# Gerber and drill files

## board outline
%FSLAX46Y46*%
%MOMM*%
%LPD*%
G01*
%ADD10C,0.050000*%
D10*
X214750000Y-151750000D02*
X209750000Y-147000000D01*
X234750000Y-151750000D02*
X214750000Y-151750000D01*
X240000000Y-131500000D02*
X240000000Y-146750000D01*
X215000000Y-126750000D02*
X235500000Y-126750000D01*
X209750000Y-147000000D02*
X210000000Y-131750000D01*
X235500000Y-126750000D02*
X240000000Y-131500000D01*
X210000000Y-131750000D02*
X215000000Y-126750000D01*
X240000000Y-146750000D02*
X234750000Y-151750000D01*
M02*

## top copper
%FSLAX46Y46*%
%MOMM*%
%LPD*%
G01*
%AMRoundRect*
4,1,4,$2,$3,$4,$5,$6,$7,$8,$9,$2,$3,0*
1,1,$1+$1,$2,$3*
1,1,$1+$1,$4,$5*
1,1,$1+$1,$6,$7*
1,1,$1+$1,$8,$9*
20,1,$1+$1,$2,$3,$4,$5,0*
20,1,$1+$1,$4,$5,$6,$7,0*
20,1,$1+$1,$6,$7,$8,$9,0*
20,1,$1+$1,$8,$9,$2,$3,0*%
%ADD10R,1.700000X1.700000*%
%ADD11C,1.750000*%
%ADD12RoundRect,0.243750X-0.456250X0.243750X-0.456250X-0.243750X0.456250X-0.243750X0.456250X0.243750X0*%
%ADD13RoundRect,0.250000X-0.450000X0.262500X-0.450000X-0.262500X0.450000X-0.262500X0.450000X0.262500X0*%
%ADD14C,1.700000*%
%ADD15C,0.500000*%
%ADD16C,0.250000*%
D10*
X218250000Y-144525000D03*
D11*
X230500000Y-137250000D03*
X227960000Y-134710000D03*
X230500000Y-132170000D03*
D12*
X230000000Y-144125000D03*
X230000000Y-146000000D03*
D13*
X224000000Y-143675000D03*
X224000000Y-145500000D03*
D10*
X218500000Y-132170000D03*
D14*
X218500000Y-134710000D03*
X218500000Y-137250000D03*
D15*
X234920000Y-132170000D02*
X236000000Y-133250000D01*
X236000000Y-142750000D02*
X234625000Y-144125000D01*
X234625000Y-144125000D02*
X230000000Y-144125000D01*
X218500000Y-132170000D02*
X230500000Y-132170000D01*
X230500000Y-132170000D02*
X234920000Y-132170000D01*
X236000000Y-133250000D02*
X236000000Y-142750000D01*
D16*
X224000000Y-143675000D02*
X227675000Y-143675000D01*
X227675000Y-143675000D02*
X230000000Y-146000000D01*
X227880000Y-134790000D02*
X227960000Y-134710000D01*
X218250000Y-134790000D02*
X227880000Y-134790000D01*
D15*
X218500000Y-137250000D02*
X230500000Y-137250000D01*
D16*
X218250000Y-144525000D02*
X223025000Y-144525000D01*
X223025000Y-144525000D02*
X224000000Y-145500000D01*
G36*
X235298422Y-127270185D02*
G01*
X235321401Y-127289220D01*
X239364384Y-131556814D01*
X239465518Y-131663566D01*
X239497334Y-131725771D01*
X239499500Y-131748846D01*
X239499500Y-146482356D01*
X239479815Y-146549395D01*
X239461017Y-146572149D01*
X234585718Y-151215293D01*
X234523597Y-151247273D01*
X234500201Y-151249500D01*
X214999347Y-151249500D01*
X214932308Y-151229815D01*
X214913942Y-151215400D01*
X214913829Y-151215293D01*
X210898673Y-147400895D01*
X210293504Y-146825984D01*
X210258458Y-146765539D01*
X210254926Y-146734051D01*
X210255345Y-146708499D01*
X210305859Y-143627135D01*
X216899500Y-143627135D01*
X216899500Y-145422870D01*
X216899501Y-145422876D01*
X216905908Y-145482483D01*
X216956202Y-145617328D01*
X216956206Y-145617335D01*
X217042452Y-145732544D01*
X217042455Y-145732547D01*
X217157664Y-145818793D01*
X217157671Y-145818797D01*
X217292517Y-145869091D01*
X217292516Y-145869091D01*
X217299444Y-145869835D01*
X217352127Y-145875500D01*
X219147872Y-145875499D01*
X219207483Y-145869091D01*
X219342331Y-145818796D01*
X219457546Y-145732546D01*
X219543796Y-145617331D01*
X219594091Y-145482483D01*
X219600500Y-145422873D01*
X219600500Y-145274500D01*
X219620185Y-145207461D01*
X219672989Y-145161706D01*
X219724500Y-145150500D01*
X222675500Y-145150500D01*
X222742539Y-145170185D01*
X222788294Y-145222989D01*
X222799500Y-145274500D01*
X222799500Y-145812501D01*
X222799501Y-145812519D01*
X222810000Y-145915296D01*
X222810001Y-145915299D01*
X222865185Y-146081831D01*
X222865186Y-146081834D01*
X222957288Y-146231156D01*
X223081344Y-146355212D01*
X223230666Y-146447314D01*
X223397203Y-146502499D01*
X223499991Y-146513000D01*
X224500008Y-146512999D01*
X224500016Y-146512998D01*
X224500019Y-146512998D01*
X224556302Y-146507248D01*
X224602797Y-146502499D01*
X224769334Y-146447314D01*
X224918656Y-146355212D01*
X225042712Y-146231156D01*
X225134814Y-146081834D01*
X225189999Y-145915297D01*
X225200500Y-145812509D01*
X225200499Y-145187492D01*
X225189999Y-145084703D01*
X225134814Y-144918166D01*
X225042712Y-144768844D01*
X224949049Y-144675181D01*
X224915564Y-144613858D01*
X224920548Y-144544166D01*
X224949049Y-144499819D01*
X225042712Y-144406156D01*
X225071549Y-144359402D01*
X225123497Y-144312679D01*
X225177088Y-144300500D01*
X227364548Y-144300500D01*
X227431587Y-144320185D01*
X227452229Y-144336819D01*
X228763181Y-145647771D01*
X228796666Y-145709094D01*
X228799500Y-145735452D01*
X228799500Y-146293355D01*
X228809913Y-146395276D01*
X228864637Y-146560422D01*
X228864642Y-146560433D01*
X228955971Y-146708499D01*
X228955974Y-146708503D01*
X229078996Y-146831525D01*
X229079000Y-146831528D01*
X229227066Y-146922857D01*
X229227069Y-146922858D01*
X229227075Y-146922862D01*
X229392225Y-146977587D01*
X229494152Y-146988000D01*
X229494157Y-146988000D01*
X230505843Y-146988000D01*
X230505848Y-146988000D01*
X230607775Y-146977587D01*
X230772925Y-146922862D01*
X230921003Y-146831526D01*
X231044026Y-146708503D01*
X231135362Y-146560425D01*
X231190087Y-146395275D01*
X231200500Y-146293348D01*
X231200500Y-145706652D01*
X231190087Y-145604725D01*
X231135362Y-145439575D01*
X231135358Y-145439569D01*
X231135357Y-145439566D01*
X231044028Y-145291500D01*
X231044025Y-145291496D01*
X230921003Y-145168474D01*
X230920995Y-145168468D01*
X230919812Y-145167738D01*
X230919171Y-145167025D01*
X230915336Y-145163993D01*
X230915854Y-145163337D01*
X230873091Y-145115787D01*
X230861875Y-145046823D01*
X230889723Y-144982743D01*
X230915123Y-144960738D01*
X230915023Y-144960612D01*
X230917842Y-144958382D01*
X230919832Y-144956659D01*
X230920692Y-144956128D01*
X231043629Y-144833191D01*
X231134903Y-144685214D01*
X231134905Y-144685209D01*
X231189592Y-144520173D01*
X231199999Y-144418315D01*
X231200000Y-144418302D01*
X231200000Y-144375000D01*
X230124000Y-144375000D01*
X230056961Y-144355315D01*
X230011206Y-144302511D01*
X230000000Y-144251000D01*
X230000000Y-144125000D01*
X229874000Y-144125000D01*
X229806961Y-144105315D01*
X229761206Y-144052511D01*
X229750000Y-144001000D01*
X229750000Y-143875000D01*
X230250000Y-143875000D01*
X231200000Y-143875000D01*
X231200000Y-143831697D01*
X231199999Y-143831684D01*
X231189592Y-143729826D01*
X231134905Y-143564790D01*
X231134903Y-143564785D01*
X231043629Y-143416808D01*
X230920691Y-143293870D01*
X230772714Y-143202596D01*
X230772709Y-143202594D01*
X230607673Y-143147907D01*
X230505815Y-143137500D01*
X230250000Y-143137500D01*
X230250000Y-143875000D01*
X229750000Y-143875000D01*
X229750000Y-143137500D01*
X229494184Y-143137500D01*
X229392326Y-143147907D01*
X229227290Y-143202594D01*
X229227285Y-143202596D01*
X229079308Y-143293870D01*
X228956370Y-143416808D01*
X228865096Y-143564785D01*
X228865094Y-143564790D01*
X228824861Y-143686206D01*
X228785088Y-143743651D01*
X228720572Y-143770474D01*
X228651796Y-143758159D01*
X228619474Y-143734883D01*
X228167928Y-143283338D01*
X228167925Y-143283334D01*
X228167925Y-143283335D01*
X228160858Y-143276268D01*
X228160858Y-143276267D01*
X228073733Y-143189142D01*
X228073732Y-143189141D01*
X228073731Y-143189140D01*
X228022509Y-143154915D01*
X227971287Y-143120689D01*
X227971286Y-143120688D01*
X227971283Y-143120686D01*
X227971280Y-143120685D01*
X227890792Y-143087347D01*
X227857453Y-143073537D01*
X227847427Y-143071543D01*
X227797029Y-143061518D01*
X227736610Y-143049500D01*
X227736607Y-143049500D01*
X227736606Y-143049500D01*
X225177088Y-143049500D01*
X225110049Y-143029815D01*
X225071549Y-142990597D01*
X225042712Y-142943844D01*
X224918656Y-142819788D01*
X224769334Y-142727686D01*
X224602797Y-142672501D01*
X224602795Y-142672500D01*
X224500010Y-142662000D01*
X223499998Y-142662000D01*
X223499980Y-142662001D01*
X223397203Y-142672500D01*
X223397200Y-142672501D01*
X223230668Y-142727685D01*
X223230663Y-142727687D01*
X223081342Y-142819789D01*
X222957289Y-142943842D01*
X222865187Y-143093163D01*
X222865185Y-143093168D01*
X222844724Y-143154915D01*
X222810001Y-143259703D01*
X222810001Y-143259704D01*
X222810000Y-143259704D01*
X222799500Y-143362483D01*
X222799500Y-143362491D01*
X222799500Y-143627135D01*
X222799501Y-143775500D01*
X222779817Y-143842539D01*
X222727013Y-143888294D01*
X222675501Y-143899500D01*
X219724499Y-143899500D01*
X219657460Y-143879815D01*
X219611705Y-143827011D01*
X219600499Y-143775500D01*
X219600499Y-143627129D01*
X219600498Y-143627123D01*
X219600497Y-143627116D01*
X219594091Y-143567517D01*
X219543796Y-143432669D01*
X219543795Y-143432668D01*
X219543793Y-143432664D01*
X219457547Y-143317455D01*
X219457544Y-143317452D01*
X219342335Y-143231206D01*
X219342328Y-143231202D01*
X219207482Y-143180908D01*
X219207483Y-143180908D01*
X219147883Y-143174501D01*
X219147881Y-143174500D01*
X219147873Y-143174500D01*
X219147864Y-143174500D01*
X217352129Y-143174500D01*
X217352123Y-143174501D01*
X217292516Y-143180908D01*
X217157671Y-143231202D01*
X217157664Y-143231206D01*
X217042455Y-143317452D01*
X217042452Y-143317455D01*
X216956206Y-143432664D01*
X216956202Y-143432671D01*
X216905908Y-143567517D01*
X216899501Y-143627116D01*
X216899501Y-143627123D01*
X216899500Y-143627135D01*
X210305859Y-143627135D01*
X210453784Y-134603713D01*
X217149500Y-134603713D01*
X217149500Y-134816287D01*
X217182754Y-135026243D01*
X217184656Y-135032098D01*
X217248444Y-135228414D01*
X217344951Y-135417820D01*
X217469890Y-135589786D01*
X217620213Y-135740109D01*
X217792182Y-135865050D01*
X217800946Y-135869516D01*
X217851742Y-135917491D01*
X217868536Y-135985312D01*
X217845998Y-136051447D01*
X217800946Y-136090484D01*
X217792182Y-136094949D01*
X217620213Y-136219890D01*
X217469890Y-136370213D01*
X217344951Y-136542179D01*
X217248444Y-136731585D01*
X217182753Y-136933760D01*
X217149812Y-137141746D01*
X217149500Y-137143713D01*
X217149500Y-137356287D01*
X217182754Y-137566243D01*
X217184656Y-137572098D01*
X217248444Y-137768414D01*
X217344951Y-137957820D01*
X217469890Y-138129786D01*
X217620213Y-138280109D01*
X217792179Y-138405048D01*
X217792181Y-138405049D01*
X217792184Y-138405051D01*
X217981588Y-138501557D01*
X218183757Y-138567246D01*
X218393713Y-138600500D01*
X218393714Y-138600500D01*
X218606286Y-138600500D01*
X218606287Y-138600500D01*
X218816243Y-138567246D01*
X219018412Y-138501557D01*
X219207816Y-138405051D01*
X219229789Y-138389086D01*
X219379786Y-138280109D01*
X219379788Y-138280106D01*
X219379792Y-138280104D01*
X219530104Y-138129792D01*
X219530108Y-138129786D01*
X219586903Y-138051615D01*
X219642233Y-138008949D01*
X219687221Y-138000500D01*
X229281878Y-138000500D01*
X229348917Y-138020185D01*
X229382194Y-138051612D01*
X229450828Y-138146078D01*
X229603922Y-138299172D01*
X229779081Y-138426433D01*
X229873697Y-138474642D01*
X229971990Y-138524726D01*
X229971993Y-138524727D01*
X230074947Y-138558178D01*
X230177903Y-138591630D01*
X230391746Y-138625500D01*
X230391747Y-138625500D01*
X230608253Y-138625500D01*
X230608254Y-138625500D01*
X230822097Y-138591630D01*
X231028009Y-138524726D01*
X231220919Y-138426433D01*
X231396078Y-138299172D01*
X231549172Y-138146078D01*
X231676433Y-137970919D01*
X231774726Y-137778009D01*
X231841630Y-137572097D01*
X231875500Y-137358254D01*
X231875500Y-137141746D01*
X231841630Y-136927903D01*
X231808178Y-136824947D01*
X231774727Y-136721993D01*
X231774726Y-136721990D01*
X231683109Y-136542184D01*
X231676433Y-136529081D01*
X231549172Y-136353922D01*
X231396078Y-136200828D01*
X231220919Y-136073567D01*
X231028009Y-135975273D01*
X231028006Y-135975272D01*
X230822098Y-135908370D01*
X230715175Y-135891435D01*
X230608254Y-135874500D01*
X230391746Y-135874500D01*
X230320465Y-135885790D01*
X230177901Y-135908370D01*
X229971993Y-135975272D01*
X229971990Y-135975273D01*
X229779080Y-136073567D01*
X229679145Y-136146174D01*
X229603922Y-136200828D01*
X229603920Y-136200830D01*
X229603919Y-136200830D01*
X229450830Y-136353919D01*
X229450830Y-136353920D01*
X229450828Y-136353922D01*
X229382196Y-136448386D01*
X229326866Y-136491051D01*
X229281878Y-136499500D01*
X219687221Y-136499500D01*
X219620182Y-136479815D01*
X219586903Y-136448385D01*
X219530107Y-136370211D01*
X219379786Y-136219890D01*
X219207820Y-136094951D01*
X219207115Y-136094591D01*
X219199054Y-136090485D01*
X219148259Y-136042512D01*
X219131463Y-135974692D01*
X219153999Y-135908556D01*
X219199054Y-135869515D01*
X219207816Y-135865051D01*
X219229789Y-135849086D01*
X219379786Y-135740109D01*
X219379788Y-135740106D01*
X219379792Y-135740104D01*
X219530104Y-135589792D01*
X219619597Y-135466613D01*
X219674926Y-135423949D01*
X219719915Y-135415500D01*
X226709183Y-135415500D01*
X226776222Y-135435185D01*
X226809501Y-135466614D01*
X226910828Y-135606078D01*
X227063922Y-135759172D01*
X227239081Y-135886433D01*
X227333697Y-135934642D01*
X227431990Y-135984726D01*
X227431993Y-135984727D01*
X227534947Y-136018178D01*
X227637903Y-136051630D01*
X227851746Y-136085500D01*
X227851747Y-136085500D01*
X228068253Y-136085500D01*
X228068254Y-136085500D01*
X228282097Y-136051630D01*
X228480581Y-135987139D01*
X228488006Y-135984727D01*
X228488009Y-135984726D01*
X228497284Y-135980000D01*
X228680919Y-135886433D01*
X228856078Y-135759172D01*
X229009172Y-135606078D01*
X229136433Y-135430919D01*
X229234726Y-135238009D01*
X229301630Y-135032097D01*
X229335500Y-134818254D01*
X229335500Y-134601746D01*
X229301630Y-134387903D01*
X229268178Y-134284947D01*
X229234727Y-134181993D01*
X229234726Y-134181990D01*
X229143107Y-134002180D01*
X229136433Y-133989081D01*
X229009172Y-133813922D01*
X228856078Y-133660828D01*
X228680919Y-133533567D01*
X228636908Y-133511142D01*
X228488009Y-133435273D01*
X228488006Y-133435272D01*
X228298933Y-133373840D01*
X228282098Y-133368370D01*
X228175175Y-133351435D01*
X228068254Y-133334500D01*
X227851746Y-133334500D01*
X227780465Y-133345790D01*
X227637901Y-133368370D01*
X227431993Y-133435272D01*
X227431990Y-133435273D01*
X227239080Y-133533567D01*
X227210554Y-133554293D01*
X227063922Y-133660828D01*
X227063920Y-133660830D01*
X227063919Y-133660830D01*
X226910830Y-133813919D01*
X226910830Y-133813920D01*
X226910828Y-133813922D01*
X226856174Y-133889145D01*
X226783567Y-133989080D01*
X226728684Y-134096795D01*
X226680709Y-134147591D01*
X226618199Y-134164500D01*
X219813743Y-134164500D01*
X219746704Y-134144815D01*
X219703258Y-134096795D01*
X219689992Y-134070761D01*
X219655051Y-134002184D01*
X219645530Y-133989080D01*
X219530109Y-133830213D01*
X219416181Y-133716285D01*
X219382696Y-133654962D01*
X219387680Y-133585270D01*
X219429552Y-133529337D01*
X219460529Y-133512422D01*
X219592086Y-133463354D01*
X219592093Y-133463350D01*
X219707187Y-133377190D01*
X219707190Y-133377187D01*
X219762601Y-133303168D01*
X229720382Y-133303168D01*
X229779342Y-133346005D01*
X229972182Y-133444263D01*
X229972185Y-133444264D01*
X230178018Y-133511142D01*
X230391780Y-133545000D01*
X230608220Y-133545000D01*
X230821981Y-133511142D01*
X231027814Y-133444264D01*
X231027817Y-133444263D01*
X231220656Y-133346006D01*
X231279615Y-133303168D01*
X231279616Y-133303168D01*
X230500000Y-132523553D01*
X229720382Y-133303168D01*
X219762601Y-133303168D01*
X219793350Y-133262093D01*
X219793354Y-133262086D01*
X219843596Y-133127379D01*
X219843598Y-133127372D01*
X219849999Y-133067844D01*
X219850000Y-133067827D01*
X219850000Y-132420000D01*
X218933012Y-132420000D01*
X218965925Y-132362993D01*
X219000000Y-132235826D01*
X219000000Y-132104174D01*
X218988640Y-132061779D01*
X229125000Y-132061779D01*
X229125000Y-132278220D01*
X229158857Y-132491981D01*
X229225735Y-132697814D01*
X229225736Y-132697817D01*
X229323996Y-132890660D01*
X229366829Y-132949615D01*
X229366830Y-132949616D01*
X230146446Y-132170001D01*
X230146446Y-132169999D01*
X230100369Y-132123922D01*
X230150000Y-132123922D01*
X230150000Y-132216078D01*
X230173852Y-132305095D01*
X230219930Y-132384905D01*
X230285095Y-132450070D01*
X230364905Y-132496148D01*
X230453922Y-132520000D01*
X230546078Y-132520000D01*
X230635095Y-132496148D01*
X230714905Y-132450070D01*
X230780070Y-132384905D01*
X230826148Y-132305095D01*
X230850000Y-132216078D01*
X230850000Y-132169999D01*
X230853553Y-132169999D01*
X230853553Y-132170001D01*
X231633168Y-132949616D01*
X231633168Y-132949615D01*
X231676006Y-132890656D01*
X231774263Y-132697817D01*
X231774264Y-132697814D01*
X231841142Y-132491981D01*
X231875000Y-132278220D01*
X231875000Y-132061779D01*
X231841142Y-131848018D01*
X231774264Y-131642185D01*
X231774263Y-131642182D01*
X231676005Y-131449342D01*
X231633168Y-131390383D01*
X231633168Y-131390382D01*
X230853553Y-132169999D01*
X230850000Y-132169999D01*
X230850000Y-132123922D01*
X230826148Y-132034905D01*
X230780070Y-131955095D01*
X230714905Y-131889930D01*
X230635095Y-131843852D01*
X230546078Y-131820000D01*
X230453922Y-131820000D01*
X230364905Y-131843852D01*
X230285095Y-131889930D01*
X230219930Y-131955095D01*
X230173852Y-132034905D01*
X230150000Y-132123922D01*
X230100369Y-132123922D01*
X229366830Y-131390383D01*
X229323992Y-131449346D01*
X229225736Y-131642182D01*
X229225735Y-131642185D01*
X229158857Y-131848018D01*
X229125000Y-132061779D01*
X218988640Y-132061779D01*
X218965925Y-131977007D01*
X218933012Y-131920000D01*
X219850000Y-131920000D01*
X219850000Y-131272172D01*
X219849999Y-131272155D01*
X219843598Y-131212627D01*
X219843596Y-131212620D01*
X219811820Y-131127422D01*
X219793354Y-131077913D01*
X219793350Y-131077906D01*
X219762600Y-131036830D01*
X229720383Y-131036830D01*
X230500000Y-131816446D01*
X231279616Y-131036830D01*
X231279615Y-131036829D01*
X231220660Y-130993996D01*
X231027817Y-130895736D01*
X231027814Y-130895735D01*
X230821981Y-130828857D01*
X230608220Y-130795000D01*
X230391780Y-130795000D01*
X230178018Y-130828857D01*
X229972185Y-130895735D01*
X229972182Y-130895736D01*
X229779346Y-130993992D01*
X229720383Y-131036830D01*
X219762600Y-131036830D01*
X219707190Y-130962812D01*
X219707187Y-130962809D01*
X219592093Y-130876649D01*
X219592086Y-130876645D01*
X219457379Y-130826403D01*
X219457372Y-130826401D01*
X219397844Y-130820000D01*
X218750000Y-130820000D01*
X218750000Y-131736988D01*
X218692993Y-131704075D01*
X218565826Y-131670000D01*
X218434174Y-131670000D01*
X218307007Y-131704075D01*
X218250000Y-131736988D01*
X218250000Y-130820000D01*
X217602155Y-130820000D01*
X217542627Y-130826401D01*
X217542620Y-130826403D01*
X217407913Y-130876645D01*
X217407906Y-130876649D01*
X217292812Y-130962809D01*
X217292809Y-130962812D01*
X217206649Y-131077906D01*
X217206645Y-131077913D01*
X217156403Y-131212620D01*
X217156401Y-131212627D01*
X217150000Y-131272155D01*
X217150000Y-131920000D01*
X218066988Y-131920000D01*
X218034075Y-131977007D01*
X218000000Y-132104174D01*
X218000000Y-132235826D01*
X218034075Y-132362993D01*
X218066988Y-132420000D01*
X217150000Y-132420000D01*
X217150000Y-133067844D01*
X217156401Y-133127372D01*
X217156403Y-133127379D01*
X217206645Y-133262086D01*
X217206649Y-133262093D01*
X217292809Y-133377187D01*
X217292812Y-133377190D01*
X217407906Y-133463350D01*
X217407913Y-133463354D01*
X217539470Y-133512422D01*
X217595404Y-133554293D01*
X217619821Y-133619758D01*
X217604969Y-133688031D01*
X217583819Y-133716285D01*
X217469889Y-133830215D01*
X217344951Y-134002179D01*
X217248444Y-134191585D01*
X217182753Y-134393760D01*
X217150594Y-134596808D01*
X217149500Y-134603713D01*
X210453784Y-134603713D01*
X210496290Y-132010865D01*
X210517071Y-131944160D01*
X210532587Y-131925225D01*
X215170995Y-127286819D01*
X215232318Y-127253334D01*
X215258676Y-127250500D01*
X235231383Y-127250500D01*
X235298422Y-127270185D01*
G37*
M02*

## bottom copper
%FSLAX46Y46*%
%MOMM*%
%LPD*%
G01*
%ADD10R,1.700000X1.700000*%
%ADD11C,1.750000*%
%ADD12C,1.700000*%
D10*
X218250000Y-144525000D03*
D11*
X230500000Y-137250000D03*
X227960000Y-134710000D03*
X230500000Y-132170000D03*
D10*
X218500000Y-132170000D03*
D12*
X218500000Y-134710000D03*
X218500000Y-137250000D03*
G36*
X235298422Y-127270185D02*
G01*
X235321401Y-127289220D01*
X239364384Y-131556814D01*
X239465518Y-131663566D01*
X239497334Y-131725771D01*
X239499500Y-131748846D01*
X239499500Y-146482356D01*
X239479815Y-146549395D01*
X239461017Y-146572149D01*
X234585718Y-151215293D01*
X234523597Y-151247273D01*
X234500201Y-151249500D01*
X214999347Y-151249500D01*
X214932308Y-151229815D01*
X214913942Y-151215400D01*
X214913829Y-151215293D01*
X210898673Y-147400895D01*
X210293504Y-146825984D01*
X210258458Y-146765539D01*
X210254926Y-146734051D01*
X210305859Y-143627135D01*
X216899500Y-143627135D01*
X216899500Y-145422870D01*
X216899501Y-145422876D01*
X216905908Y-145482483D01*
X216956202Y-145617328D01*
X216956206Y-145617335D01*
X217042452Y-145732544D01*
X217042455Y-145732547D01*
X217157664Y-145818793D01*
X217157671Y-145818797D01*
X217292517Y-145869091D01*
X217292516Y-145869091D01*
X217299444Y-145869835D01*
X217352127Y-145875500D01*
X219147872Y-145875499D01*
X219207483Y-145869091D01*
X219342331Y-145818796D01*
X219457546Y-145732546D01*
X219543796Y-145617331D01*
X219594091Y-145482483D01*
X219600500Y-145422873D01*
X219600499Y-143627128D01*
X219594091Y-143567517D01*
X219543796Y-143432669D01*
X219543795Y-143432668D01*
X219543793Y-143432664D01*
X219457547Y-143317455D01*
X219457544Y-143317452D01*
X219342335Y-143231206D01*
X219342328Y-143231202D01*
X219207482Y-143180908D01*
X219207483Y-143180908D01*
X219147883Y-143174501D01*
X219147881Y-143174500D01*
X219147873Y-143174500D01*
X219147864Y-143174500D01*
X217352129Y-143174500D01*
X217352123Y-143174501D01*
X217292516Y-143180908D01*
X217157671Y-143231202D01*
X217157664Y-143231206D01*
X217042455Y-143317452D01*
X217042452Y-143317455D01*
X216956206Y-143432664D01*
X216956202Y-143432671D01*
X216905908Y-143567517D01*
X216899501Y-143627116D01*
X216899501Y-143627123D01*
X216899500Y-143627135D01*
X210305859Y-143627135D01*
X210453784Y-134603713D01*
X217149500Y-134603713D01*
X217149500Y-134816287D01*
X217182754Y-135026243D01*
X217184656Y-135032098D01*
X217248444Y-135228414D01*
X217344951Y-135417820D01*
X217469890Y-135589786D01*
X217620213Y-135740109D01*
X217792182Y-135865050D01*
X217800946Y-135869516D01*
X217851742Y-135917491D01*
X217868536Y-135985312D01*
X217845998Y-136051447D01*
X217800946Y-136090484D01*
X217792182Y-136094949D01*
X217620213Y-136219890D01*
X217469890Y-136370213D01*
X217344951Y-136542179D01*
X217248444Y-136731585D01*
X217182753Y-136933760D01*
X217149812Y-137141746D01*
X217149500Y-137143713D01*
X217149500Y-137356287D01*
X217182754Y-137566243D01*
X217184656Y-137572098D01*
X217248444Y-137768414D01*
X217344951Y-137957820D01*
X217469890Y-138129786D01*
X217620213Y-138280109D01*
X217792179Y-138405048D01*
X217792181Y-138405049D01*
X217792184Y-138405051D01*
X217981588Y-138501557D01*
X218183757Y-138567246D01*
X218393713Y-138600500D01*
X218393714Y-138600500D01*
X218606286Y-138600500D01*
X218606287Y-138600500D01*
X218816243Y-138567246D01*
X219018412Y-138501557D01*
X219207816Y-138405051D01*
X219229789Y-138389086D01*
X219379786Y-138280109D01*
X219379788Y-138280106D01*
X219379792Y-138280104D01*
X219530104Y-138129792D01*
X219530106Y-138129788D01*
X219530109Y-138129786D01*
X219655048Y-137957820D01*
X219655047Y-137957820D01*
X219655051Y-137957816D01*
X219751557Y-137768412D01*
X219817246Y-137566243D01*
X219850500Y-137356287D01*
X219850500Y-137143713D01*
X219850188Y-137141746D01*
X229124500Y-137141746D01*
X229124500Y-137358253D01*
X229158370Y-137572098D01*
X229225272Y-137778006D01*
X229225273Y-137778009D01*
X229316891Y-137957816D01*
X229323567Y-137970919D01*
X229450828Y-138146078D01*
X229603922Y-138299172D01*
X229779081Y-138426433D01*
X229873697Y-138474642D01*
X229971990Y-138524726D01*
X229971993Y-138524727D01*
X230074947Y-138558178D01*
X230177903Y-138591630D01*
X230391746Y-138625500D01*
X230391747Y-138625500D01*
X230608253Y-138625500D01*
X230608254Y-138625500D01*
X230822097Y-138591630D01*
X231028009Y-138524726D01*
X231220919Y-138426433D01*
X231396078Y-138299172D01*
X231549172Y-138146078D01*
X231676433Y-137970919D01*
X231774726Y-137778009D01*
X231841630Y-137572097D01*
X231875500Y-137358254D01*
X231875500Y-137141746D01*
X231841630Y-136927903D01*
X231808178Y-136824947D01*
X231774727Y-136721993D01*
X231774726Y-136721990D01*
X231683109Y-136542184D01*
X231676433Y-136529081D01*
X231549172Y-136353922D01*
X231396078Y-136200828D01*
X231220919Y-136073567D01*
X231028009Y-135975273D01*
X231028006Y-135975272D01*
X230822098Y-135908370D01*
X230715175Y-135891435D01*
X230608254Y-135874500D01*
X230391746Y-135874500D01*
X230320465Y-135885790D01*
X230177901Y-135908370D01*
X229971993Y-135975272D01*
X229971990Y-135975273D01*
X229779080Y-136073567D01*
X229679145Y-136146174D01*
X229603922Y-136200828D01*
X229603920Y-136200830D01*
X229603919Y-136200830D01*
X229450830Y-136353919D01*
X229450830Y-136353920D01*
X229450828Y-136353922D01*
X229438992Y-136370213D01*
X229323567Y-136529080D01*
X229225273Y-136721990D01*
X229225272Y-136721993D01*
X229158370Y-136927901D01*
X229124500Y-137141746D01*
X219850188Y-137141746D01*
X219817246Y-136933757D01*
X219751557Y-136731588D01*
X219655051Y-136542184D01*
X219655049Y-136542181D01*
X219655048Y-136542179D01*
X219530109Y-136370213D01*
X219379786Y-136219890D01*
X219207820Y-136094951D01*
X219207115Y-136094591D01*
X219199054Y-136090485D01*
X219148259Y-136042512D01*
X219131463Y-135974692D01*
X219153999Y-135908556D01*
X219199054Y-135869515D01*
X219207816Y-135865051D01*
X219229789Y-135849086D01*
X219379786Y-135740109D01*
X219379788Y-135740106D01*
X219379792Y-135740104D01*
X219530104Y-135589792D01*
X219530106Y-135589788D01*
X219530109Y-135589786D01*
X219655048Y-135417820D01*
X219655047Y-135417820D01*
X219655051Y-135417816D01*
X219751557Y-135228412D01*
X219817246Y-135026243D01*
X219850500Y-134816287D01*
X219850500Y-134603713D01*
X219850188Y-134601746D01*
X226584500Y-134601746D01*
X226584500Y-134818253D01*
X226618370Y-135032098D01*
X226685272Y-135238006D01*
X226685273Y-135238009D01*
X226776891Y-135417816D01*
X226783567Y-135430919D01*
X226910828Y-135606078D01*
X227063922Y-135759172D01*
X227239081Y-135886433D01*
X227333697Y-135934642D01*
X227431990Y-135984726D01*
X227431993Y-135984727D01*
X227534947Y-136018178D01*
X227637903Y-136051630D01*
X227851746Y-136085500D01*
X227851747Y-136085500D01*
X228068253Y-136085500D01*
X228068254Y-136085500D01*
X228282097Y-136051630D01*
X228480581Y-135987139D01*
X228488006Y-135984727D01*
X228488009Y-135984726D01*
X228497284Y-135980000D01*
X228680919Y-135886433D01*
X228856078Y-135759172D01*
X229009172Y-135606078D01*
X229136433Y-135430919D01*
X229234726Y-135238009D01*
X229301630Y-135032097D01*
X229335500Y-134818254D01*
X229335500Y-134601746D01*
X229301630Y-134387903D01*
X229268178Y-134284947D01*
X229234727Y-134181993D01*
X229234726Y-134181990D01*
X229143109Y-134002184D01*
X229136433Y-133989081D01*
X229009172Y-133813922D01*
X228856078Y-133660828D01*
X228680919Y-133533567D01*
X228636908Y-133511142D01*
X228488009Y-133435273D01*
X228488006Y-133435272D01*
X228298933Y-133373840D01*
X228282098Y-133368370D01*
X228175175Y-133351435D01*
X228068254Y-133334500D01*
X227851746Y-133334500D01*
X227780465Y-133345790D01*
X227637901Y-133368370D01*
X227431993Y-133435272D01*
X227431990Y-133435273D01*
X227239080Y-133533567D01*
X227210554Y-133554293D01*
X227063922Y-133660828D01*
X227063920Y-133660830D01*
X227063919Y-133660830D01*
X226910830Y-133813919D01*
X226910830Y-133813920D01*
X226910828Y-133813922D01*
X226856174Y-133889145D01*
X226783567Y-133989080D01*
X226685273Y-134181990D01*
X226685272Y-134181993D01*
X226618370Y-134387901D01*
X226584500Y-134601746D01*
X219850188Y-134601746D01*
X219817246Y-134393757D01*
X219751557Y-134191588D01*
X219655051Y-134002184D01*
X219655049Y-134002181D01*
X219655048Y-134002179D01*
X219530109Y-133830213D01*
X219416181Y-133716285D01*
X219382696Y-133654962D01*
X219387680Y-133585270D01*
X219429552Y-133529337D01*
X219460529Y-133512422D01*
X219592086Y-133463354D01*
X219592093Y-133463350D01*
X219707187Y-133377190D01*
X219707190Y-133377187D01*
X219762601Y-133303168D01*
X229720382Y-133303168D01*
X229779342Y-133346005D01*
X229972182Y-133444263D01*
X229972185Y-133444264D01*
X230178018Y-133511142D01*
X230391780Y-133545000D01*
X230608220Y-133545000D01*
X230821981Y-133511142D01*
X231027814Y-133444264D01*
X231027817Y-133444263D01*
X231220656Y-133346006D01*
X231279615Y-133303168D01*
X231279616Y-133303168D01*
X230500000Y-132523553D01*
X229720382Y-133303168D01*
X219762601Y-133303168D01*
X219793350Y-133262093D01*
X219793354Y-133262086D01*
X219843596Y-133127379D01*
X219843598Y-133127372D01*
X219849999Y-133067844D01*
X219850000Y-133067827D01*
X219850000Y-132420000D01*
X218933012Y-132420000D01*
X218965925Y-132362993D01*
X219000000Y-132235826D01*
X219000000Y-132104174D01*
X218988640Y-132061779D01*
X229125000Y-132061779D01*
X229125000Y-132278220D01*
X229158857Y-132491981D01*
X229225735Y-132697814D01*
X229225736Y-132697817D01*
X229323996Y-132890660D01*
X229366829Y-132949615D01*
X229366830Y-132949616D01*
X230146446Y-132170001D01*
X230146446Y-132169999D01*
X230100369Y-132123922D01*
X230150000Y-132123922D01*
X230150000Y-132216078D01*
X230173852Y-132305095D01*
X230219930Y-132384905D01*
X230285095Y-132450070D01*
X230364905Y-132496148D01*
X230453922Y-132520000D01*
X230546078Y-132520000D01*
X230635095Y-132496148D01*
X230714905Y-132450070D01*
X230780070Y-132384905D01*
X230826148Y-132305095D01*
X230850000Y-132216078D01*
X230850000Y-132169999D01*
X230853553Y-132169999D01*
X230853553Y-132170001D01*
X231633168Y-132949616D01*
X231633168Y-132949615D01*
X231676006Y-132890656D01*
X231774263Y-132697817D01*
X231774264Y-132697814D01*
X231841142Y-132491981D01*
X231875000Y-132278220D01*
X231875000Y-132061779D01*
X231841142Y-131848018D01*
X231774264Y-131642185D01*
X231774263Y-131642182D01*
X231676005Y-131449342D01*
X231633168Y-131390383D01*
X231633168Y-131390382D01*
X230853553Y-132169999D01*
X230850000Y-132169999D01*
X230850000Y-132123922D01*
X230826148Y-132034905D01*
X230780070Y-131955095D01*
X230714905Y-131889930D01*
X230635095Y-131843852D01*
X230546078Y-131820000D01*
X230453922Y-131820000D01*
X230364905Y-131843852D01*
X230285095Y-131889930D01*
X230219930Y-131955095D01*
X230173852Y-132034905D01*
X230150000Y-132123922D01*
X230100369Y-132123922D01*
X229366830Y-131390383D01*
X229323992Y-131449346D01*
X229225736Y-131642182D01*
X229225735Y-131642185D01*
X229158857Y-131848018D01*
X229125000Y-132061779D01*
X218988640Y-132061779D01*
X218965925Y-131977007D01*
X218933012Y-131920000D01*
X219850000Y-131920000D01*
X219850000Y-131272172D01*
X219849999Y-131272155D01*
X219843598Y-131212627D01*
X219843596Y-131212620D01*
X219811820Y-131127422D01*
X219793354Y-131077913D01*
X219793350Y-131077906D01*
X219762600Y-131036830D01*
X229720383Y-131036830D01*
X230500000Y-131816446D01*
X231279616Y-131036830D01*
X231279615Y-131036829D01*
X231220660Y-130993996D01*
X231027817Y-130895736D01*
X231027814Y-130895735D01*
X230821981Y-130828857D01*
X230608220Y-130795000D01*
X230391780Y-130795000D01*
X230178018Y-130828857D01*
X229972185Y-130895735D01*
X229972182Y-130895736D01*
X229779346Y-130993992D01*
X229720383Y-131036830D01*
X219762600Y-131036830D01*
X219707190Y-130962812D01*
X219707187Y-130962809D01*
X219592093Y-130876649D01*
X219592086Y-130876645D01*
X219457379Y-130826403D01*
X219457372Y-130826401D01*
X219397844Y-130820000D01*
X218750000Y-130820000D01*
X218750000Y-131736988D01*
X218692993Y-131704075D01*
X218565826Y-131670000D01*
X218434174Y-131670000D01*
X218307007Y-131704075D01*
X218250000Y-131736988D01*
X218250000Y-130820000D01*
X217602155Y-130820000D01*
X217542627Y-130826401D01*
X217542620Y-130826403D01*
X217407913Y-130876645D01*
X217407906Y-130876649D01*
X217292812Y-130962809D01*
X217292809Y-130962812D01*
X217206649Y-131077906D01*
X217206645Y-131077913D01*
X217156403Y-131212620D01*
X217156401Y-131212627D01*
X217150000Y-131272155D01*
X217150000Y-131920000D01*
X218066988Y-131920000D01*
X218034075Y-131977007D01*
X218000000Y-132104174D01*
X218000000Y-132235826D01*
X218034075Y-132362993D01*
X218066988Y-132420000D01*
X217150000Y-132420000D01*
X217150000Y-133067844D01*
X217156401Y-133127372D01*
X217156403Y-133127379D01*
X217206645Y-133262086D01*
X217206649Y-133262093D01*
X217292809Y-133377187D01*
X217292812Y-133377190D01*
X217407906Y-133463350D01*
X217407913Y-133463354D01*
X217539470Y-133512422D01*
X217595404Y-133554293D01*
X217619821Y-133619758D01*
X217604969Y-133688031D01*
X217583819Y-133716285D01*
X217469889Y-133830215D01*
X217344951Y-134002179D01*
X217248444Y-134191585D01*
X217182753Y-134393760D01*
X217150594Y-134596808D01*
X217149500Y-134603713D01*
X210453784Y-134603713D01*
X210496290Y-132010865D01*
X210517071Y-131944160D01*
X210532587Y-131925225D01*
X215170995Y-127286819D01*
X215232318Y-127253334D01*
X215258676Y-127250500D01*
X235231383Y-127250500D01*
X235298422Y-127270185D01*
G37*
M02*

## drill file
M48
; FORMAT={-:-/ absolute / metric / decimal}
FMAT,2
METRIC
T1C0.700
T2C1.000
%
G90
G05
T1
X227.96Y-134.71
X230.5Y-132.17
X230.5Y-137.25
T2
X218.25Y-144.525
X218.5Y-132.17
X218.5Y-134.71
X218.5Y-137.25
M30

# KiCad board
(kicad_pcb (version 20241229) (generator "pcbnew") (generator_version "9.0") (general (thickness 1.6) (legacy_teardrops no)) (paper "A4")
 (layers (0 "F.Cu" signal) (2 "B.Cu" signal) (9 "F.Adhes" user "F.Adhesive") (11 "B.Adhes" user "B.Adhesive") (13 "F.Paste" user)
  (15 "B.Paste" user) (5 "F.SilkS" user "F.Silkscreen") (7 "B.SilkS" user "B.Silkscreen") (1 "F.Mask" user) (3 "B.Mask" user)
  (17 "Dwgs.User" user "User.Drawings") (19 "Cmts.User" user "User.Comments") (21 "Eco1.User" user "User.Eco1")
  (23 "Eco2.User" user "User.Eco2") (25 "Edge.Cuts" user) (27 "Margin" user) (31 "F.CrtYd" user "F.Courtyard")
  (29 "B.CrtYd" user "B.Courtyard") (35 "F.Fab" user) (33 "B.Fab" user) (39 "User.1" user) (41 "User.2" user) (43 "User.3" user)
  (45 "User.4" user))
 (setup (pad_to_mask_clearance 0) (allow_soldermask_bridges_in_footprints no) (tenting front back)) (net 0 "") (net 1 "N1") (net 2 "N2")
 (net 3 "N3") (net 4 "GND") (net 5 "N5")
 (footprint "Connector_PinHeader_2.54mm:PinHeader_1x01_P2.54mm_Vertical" (layer "F.Cu") (at 218.25 144.525)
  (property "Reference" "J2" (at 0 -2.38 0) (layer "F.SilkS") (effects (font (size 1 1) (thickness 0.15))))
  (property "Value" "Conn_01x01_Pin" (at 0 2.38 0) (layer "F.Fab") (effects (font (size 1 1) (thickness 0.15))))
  (pad "1" thru_hole rect (at 0 0) (size 1.7 1.7) (drill 1) (layers "*.Cu" "*.Mask") (remove_unused_layers no) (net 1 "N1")))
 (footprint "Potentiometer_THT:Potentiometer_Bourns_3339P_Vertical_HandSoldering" (layer "F.Cu") (at 230.5 137.25)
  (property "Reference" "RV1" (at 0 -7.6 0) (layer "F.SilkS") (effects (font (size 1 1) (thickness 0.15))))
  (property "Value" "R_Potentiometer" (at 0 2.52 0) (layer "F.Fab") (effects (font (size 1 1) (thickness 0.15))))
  (pad "1" thru_hole circle (at 0 0) (size 1.75 1.75) (drill 0.7) (layers "*.Cu" "*.Mask") (remove_unused_layers no) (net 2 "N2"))
  (pad "2" thru_hole circle (at -2.54 -2.54) (size 1.75 1.75) (drill 0.7) (layers "*.Cu" "*.Mask") (remove_unused_layers no) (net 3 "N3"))
  (pad "3" thru_hole circle (at 0 -5.08) (size 1.75 1.75) (drill 0.7) (layers "*.Cu" "*.Mask") (remove_unused_layers no) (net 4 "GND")))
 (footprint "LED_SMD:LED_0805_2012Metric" (layer "F.Cu") (at 230 145.0625 -90)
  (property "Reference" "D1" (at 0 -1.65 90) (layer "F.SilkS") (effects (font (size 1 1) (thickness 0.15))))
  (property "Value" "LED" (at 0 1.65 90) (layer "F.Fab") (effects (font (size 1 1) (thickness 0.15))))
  (pad "1" smd roundrect (at -0.9375 0 270) (size 0.975 1.4) (layers "F.Cu" "F.Mask" "F.Paste") (roundrect_rratio 0.25) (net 4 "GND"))
  (pad "2" smd roundrect (at 0.9375 0 270) (size 0.975 1.4) (layers "F.Cu" "F.Mask" "F.Paste") (roundrect_rratio 0.25) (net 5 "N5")))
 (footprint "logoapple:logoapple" (layer "F.Cu") (at 234.25 147.75)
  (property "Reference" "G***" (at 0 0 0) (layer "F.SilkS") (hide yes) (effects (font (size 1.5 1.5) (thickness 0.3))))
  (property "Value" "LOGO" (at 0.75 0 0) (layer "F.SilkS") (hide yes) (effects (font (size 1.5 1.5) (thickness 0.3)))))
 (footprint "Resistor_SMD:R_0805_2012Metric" (layer "F.Cu") (at 224 144.5875 -90)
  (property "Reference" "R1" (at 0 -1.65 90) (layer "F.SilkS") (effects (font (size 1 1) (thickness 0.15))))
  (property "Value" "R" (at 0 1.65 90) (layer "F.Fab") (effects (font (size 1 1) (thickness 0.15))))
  (pad "1" smd roundrect (at -0.9125 0 270) (size 1.025 1.4) (layers "F.Cu" "F.Mask" "F.Paste") (roundrect_rratio 0.243902) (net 5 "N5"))
  (pad "2" smd roundrect (at 0.9125 0 270) (size 1.025 1.4) (layers "F.Cu" "F.Mask" "F.Paste") (roundrect_rratio 0.243902) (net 1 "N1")))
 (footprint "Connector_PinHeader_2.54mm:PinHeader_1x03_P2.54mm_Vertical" (layer "F.Cu") (at 218.5 132.17)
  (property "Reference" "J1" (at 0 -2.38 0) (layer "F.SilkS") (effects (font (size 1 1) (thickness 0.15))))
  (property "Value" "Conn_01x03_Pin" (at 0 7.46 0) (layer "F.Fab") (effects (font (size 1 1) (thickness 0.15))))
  (pad "1" thru_hole rect (at 0 0) (size 1.7 1.7) (drill 1) (layers "*.Cu" "*.Mask") (remove_unused_layers no) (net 4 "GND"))
  (pad "2" thru_hole circle (at 0 2.54) (size 1.7 1.7) (drill 1) (layers "*.Cu" "*.Mask") (remove_unused_layers no) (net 3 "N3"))
  (pad "3" thru_hole circle (at 0 5.08) (size 1.7 1.7) (drill 1) (layers "*.Cu" "*.Mask") (remove_unused_layers no) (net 2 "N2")))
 (gr_line (start 214.75 151.75) (end 209.75 147) (stroke (width 0.05) (type default)) (layer "Edge.Cuts"))
 (gr_line (start 234.75 151.75) (end 214.75 151.75) (stroke (width 0.05) (type default)) (layer "Edge.Cuts"))
 (gr_line (start 240 131.5) (end 240 146.75) (stroke (width 0.05) (type default)) (layer "Edge.Cuts"))
 (gr_line (start 215 126.75) (end 235.5 126.75) (stroke (width 0.05) (type default)) (layer "Edge.Cuts"))
 (gr_line (start 209.75 147) (end 210 131.75) (stroke (width 0.05) (type default)) (layer "Edge.Cuts"))
 (gr_line (start 235.5 126.75) (end 240 131.5) (stroke (width 0.05) (type default)) (layer "Edge.Cuts"))
 (gr_line (start 210 131.75) (end 215 126.75) (stroke (width 0.05) (type default)) (layer "Edge.Cuts"))
 (gr_line (start 240 146.75) (end 234.75 151.75) (stroke (width 0.05) (type default)) (layer "Edge.Cuts"))
 (segment (start 234.92 132.17) (end 236 133.25) (width 0.5) (layer "F.Cu") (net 4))
 (segment (start 236 142.75) (end 234.625 144.125) (width 0.5) (layer "F.Cu") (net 4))
 (segment (start 234.625 144.125) (end 230 144.125) (width 0.5) (layer "F.Cu") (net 4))
 (segment (start 218.5 132.17) (end 230.5 132.17) (width 0.5) (layer "F.Cu") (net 4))
 (segment (start 230.5 132.17) (end 234.92 132.17) (width 0.5) (layer "F.Cu") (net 4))
 (segment (start 236 133.25) (end 236 142.75) (width 0.5) (layer "F.Cu") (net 4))
 (segment (start 224 143.675) (end 227.675 143.675) (width 0.25) (layer "F.Cu") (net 5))
 (segment (start 227.675 143.675) (end 230 146) (width 0.25) (layer "F.Cu") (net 5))
 (segment (start 227.88 134.79) (end 227.96 134.71) (width 0.25) (layer "F.Cu") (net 3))
 (segment (start 218.25 134.79) (end 227.88 134.79) (width 0.25) (layer "F.Cu") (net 3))
 (segment (start 218.5 137.25) (end 230.5 137.25) (width 0.5) (layer "F.Cu") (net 2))
 (segment (start 218.25 144.525) (end 223.025 144.525) (width 0.25) (layer "F.Cu") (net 1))
 (segment (start 223.025 144.525) (end 224 145.5) (width 0.25) (layer "F.Cu") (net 1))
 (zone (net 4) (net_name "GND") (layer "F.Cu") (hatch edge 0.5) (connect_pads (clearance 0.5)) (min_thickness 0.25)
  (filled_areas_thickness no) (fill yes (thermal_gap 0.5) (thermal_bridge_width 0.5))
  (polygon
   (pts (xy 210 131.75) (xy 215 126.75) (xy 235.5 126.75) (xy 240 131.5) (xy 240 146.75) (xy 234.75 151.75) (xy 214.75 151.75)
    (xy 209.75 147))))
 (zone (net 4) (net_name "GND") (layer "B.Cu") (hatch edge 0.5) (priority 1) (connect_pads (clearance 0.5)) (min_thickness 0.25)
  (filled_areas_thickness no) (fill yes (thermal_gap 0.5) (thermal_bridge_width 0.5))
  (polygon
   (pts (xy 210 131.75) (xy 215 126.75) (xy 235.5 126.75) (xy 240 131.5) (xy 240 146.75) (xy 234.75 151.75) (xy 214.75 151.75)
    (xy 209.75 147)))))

